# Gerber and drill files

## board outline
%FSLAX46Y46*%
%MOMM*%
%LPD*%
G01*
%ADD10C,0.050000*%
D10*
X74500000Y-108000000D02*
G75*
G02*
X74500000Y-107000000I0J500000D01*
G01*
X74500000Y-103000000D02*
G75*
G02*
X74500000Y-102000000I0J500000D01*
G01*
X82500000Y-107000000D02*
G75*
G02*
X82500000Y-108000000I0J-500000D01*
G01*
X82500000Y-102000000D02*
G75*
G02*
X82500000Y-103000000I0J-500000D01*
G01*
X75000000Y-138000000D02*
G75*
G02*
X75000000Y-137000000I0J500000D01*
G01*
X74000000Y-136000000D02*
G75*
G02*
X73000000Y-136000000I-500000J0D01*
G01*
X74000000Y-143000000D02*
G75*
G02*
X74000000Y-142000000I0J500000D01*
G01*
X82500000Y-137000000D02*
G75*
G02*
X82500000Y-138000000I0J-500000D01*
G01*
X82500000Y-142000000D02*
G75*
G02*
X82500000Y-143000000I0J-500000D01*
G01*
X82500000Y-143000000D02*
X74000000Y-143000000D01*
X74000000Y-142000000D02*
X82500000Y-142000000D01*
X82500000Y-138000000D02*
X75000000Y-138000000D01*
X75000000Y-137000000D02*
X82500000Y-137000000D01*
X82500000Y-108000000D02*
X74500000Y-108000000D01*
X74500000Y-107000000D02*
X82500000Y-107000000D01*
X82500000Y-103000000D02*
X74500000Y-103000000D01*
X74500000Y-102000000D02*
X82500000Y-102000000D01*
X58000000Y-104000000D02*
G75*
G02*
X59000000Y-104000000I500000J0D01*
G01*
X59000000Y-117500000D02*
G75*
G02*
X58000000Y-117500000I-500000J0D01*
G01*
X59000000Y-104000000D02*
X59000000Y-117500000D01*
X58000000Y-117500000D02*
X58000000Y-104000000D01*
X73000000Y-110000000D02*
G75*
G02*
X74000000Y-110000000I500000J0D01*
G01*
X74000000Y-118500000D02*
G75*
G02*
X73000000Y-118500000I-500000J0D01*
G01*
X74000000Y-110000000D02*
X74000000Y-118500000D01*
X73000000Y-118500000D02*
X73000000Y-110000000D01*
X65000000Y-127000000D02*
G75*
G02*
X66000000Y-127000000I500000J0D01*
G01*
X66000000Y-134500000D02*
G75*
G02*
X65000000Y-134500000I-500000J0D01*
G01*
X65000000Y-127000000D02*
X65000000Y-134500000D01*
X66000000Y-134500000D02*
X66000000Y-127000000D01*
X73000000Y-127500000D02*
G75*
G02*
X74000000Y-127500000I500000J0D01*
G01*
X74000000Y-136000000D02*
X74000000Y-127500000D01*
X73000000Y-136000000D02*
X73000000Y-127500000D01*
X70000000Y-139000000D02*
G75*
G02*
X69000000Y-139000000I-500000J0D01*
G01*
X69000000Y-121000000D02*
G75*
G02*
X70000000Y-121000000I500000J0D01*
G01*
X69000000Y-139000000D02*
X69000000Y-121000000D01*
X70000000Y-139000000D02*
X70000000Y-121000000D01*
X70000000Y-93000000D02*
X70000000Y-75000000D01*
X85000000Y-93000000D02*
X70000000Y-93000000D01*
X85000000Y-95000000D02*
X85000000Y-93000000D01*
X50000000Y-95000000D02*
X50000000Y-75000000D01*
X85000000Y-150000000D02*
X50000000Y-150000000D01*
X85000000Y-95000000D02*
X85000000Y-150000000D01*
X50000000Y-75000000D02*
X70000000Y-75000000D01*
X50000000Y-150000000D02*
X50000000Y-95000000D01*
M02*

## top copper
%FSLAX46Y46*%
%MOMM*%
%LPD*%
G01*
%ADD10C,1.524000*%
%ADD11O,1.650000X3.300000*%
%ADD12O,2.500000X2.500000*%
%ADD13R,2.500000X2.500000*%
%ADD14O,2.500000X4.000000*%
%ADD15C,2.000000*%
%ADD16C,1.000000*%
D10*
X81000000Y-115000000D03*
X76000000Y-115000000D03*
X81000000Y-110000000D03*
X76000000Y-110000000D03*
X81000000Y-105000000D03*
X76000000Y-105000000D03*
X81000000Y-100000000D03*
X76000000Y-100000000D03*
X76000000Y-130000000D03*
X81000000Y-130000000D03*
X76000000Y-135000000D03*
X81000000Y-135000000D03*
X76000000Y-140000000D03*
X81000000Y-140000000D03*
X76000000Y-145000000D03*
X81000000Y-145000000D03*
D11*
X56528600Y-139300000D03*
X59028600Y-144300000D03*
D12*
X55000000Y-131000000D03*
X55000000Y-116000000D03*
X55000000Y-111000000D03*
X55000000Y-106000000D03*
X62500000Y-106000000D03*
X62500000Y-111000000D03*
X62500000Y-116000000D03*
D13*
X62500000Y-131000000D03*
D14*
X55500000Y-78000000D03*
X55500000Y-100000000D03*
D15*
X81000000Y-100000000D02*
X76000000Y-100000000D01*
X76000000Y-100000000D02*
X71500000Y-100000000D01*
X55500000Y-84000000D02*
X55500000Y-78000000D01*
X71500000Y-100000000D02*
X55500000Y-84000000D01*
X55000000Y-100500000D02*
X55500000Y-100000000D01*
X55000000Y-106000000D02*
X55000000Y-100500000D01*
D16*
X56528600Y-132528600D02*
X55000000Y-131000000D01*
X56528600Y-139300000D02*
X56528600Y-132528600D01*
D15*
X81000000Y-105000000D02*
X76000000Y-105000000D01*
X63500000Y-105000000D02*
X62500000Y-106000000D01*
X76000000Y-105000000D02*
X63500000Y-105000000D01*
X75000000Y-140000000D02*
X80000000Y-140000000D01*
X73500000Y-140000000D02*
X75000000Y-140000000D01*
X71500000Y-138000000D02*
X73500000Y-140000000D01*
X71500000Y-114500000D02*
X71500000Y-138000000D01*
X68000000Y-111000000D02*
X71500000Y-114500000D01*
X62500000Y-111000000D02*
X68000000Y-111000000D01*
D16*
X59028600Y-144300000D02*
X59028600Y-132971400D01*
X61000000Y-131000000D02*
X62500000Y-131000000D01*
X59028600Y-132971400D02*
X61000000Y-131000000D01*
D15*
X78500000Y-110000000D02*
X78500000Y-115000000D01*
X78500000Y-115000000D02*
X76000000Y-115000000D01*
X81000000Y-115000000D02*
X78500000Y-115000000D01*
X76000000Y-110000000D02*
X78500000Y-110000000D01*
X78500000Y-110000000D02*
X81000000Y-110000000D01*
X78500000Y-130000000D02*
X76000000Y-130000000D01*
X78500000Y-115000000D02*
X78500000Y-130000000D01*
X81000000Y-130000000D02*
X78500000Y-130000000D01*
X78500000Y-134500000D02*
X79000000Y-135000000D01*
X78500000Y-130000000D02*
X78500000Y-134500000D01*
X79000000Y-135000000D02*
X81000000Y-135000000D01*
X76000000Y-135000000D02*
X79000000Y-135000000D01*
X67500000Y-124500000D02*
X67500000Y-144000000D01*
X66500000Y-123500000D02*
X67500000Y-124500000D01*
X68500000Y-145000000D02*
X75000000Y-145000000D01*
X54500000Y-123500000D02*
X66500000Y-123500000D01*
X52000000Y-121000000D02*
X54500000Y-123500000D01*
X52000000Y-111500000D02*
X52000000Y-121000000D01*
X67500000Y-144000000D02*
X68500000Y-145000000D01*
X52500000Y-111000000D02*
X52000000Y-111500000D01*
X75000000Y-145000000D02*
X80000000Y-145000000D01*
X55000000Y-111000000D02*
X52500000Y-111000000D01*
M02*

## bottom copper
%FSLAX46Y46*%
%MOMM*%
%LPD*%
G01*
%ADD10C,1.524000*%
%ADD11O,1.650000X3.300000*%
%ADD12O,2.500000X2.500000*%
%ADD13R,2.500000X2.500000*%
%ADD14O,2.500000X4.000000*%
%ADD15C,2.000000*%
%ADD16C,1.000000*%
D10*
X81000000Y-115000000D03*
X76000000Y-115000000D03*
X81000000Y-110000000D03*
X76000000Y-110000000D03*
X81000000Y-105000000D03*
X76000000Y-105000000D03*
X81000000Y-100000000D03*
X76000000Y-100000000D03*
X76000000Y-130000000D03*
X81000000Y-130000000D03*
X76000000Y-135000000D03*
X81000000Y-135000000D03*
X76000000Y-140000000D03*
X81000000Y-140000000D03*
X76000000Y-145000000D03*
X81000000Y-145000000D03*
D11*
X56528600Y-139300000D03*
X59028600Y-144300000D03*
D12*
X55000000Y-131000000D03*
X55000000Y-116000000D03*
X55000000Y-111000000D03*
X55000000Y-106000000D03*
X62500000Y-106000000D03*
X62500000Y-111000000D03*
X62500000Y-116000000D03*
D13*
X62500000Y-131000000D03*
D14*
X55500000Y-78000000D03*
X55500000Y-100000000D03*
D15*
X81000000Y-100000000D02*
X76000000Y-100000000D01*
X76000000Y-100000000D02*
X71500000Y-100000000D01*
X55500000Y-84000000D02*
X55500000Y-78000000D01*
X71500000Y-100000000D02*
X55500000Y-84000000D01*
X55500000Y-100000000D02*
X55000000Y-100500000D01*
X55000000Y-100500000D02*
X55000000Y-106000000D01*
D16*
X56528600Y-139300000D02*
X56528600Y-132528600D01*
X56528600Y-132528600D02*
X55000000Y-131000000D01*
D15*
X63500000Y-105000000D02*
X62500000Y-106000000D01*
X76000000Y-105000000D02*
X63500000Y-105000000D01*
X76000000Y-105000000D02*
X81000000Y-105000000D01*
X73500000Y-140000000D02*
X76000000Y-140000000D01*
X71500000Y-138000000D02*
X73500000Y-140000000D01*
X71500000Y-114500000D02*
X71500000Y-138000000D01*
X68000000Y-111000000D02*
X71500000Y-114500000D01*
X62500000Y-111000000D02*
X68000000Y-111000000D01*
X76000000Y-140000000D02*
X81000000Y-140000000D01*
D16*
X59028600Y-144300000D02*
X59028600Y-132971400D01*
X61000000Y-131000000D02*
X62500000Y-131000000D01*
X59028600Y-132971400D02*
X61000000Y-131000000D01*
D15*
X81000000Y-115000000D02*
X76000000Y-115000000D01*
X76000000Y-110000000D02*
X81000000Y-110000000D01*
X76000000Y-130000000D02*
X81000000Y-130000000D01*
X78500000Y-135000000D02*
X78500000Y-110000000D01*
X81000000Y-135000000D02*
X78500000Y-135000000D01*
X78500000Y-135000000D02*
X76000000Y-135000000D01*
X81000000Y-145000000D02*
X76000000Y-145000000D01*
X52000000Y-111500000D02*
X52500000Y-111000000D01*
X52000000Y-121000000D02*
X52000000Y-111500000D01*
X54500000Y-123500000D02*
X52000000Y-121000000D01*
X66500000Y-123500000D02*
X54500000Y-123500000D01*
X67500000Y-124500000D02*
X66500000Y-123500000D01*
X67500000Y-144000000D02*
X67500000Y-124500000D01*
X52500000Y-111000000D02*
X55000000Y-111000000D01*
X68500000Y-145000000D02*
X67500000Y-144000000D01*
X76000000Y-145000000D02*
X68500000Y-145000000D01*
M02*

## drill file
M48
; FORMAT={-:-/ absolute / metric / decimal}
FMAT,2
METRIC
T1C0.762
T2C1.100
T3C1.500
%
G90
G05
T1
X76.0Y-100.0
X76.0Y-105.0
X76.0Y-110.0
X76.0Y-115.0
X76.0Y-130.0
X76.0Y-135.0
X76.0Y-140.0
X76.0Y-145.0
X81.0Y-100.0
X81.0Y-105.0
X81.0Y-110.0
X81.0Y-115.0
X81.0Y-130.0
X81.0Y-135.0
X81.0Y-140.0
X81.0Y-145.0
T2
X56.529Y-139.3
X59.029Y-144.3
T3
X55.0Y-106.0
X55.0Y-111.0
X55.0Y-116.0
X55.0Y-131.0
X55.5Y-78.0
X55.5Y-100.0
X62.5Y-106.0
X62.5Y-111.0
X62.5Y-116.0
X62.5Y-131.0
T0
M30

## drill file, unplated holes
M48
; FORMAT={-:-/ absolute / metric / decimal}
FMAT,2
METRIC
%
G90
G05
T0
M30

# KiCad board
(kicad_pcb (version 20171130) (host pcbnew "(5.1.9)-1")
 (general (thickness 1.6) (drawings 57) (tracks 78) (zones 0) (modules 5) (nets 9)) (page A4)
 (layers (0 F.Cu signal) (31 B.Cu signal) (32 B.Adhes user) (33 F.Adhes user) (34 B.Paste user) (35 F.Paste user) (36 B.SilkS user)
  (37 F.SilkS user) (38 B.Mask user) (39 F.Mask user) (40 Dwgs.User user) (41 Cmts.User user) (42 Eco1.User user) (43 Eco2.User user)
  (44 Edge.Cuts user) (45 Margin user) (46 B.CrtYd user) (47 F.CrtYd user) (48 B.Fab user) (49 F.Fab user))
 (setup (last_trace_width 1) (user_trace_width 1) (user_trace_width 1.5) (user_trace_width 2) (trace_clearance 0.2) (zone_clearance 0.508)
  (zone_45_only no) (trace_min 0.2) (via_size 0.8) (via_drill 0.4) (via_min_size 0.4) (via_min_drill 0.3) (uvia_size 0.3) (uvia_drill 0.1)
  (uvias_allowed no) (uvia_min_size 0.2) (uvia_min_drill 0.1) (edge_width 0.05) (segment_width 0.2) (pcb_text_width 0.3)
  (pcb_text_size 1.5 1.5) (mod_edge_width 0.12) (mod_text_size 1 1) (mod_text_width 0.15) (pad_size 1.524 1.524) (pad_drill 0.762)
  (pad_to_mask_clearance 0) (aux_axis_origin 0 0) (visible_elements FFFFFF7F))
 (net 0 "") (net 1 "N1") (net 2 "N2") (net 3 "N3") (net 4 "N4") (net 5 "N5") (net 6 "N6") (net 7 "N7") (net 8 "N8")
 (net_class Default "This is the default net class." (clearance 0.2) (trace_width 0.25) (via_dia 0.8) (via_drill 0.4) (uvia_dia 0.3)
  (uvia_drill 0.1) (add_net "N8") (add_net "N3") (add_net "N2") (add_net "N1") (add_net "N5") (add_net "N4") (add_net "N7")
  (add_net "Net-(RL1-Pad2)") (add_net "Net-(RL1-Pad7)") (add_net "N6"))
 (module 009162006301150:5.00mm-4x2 (layer F.Cu) (at 76 100 270)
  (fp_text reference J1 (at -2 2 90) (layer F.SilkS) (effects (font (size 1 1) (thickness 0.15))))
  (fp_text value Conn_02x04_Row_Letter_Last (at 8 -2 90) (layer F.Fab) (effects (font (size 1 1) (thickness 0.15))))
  (pad 4b thru_hole circle (at 15 -5 270) (size 1.524 1.524) (drill 0.762) (layers *.Cu *.Mask) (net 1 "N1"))
  (pad 4a thru_hole circle (at 15 0 270) (size 1.524 1.524) (drill 0.762) (layers *.Cu *.Mask) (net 1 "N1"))
  (pad 3b thru_hole circle (at 10 -5 270) (size 1.524 1.524) (drill 0.762) (layers *.Cu *.Mask) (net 1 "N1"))
  (pad 3a thru_hole circle (at 10 0 270) (size 1.524 1.524) (drill 0.762) (layers *.Cu *.Mask) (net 1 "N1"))
  (pad 2b thru_hole circle (at 5 -5 270) (size 1.524 1.524) (drill 0.762) (layers *.Cu *.Mask) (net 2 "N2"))
  (pad 2a thru_hole circle (at 5 0 270) (size 1.524 1.524) (drill 0.762) (layers *.Cu *.Mask) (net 2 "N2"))
  (pad 1b thru_hole circle (at 0 -5 270) (size 1.524 1.524) (drill 0.762) (layers *.Cu *.Mask) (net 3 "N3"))
  (pad 1a thru_hole circle (at 0 0 270) (size 1.524 1.524) (drill 0.762) (layers *.Cu *.Mask) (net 3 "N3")))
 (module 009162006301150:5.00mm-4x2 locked (layer F.Cu) (at 81 145 90)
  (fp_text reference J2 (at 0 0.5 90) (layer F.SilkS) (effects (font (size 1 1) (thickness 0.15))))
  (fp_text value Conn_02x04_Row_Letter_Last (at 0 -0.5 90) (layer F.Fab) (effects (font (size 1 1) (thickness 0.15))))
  (pad 4b thru_hole circle (at 15 -5 90) (size 1.524 1.524) (drill 0.762) (layers *.Cu *.Mask) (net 1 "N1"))
  (pad 4a thru_hole circle (at 15 0 90) (size 1.524 1.524) (drill 0.762) (layers *.Cu *.Mask) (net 1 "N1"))
  (pad 3b thru_hole circle (at 10 -5 90) (size 1.524 1.524) (drill 0.762) (layers *.Cu *.Mask) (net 1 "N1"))
  (pad 3a thru_hole circle (at 10 0 90) (size 1.524 1.524) (drill 0.762) (layers *.Cu *.Mask) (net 1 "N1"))
  (pad 2b thru_hole circle (at 5 -5 90) (size 1.524 1.524) (drill 0.762) (layers *.Cu *.Mask) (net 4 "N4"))
  (pad 2a thru_hole circle (at 5 0 90) (size 1.524 1.524) (drill 0.762) (layers *.Cu *.Mask) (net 4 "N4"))
  (pad 1b thru_hole circle (at 0 -5 90) (size 1.524 1.524) (drill 0.762) (layers *.Cu *.Mask) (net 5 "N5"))
  (pad 1a thru_hole circle (at 0 0 90) (size 1.524 1.524) (drill 0.762) (layers *.Cu *.Mask) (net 5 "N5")))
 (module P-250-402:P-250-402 (layer F.Cu) (at 57 143 270)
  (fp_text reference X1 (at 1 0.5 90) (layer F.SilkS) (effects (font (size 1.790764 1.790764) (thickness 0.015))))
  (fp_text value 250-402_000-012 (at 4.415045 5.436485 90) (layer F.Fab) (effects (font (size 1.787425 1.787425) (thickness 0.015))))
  (pad L2 thru_hole oval (at -3.7 0.4714 270) (size 3.3 1.65) (drill 1.1) (layers *.Cu *.Mask) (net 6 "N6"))
  (pad L1 thru_hole oval (at 1.3 -2.0286 270) (size 3.3 1.65) (drill 1.1) (layers *.Cu *.Mask) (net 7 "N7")))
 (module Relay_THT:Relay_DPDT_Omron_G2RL (layer F.Cu) (at 62.5 131 90)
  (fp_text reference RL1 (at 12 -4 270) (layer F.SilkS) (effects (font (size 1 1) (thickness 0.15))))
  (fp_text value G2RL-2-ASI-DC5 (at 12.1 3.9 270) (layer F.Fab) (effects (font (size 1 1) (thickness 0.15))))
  (pad 8 thru_hole oval (at 0 -7.5 180) (size 2.5 2.5) (drill 1.5) (layers *.Cu *.Mask) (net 6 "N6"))
  (pad 7 thru_hole oval (at 15 -7.5 180) (size 2.5 2.5) (drill 1.5) (layers *.Cu *.Mask))
  (pad 6 thru_hole oval (at 20 -7.5 180) (size 2.5 2.5) (drill 1.5) (layers *.Cu *.Mask) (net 5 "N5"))
  (pad 5 thru_hole oval (at 25 -7.5 180) (size 2.5 2.5) (drill 1.5) (layers *.Cu *.Mask) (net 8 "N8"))
  (pad 4 thru_hole oval (at 25 0 180) (size 2.5 2.5) (drill 1.5) (layers *.Cu *.Mask) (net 2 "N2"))
  (pad 3 thru_hole oval (at 20 0 180) (size 2.5 2.5) (drill 1.5) (layers *.Cu *.Mask) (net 4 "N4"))
  (pad 2 thru_hole oval (at 15 0 180) (size 2.5 2.5) (drill 1.5) (layers *.Cu *.Mask))
  (pad 1 thru_hole rect (at 0 0 180) (size 2.5 2.5) (drill 1.5) (layers *.Cu *.Mask) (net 7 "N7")))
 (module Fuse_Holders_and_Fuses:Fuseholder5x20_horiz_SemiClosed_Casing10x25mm (layer F.Cu) (at 55.5 100 90)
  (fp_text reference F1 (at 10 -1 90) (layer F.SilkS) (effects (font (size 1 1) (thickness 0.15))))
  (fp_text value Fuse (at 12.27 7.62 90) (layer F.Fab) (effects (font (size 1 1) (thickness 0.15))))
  (pad 2 thru_hole oval (at 22 0) (size 2.5 4) (drill 1.5) (layers *.Cu *.Mask) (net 3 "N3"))
  (pad 1 thru_hole oval (at 0 0) (size 2.5 4) (drill 1.5) (layers *.Cu *.Mask) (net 8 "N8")))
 (gr_arc (start 74.5 107.5) (end 74.5 107) (angle -180) (layer Edge.Cuts) (width 0.05))
 (gr_arc (start 74.5 102.5) (end 74.5 102) (angle -180) (layer Edge.Cuts) (width 0.05))
 (gr_arc (start 82.5 107.5) (end 82.5 108) (angle -180) (layer Edge.Cuts) (width 0.05))
 (gr_arc (start 82.5 102.5) (end 82.5 103) (angle -180) (layer Edge.Cuts) (width 0.05))
 (gr_arc (start 75 137.5) (end 75 137) (angle -180) (layer Edge.Cuts) (width 0.05))
 (gr_arc (start 73.5 136) (end 73 136) (angle -180) (layer Edge.Cuts) (width 0.05))
 (gr_arc (start 74 142.5) (end 74 142) (angle -180) (layer Edge.Cuts) (width 0.05))
 (gr_arc (start 82.5 137.5) (end 82.5 138) (angle -180) (layer Edge.Cuts) (width 0.05))
 (gr_arc (start 82.5 142.5) (end 82.5 143) (angle -180) (layer Edge.Cuts) (width 0.05))
 (gr_line (start 82.5 143) (end 74 143) (layer Edge.Cuts) (width 0.05))
 (gr_line (start 74 142) (end 82.5 142) (layer Edge.Cuts) (width 0.05))
 (gr_line (start 82.5 138) (end 75 138) (layer Edge.Cuts) (width 0.05))
 (gr_line (start 75 137) (end 82.5 137) (layer Edge.Cuts) (width 0.05))
 (gr_line (start 82.5 108) (end 74.5 108) (layer Edge.Cuts) (width 0.05))
 (gr_line (start 74.5 107) (end 82.5 107) (layer Edge.Cuts) (width 0.05))
 (gr_line (start 82.5 103) (end 74.5 103) (layer Edge.Cuts) (width 0.05))
 (gr_line (start 74.5 102) (end 82.5 102) (layer Edge.Cuts) (width 0.05))
 (gr_arc (start 58.5 104) (end 59 104) (angle -180) (layer Edge.Cuts) (width 0.05))
 (gr_arc (start 58.5 117.5) (end 58 117.5) (angle -180) (layer Edge.Cuts) (width 0.05))
 (gr_line (start 59 104) (end 59 117.5) (layer Edge.Cuts) (width 0.05))
 (gr_line (start 58 117.5) (end 58 104) (layer Edge.Cuts) (width 0.05))
 (gr_arc (start 73.5 110) (end 74 110) (angle -180) (layer Edge.Cuts) (width 0.05))
 (gr_arc (start 73.5 118.5) (end 73 118.5) (angle -180) (layer Edge.Cuts) (width 0.05))
 (gr_line (start 74 110) (end 74 118.5) (layer Edge.Cuts) (width 0.05))
 (gr_line (start 73 118.5) (end 73 110) (layer Edge.Cuts) (width 0.05))
 (gr_arc (start 65.5 127) (end 66 127) (angle -180) (layer Edge.Cuts) (width 0.05))
 (gr_arc (start 65.5 134.5) (end 65 134.5) (angle -180) (layer Edge.Cuts) (width 0.05))
 (gr_line (start 65 127) (end 65 134.5) (layer Edge.Cuts) (width 0.05))
 (gr_line (start 66 134.5) (end 66 127) (layer Edge.Cuts) (width 0.05))
 (gr_arc (start 73.5 127.5) (end 74 127.5) (angle -180) (layer Edge.Cuts) (width 0.05))
 (gr_line (start 74 136) (end 74 127.5) (layer Edge.Cuts) (width 0.05))
 (gr_line (start 73 136) (end 73 127.5) (layer Edge.Cuts) (width 0.05))
 (gr_arc (start 69.5 139) (end 69 139) (angle -180) (layer Edge.Cuts) (width 0.05))
 (gr_arc (start 69.5 121) (end 70 121) (angle -180) (layer Edge.Cuts) (width 0.05))
 (gr_line (start 69 139) (end 69 121) (layer Edge.Cuts) (width 0.05))
 (gr_line (start 70 139) (end 70 121) (layer Edge.Cuts) (width 0.05))
 (gr_line (start 70 93) (end 70 75) (layer Edge.Cuts) (width 0.05))
 (gr_line (start 85 93) (end 70 93) (layer Edge.Cuts) (width 0.05))
 (gr_line (start 85 95) (end 85 93) (layer Edge.Cuts) (width 0.05))
 (gr_line (start 50 95) (end 50 75) (layer Edge.Cuts) (width 0.05))
 (gr_line (start 85 150) (end 50 150) (layer Edge.Cuts) (width 0.05))
 (gr_line (start 85 95) (end 85 150) (layer Edge.Cuts) (width 0.05))
 (gr_line (start 50 75) (end 70 75) (layer Edge.Cuts) (width 0.05))
 (gr_line (start 50 150) (end 50 95) (layer Edge.Cuts) (width 0.05))
 (segment (start 81 100) (end 76 100) (width 2) (layer B.Cu) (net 3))
 (segment (start 76 100) (end 71.5 100) (width 2) (layer B.Cu) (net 3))
 (segment (start 55.5 84) (end 55.5 78) (width 2) (layer B.Cu) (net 3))
 (segment (start 71.5 100) (end 55.5 84) (width 2) (layer B.Cu) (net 3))
 (segment (start 81 100) (end 76 100) (width 2) (layer F.Cu) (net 3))
 (segment (start 76 100) (end 71.5 100) (width 2) (layer F.Cu) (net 3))
 (segment (start 55.5 84) (end 55.5 78) (width 2) (layer F.Cu) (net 3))
 (segment (start 71.5 100) (end 55.5 84) (width 2) (layer F.Cu) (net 3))
 (segment (start 55.5 100) (end 55 100.5) (width 2) (layer B.Cu) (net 8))
 (segment (start 55 100.5) (end 55 106) (width 2) (layer B.Cu) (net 8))
 (segment (start 55 100.5) (end 55.5 100) (width 2) (layer F.Cu) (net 8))
 (segment (start 55 106) (end 55 100.5) (width 2) (layer F.Cu) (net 8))
 (segment (start 56.5286 139.3) (end 56.5286 132.5286) (width 1) (layer B.Cu) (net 6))
 (segment (start 56.5286 132.5286) (end 55 131) (width 1) (layer B.Cu) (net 6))
 (segment (start 56.5286 132.5286) (end 55 131) (width 1) (layer F.Cu) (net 6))
 (segment (start 56.5286 139.3) (end 56.5286 132.5286) (width 1) (layer F.Cu) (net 6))
 (segment (start 63.5 105) (end 62.5 106) (width 2) (layer B.Cu) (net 2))
 (segment (start 76 105) (end 63.5 105) (width 2) (layer B.Cu) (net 2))
 (segment (start 81 105) (end 76 105) (width 2) (layer F.Cu) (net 2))
 (segment (start 63.5 105) (end 62.5 106) (width 2) (layer F.Cu) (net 2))
 (segment (start 76 105) (end 63.5 105) (width 2) (layer F.Cu) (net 2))
 (segment (start 76 105) (end 81 105) (width 2) (layer B.Cu) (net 2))
 (segment (start 75 140) (end 80 140) (width 2) (layer F.Cu) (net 4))
 (segment (start 73.5 140) (end 75 140) (width 2) (layer F.Cu) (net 4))
 (segment (start 71.5 138) (end 73.5 140) (width 2) (layer F.Cu) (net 4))
 (segment (start 71.5 114.5) (end 71.5 138) (width 2) (layer F.Cu) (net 4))
 (segment (start 68 111) (end 71.5 114.5) (width 2) (layer F.Cu) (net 4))
 (segment (start 62.5 111) (end 68 111) (width 2) (layer F.Cu) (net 4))
 (segment (start 73.5 140) (end 76 140) (width 2) (layer B.Cu) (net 4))
 (segment (start 71.5 138) (end 73.5 140) (width 2) (layer B.Cu) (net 4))
 (segment (start 71.5 114.5) (end 71.5 138) (width 2) (layer B.Cu) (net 4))
 (segment (start 68 111) (end 71.5 114.5) (width 2) (layer B.Cu) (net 4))
 (segment (start 62.5 111) (end 68 111) (width 2) (layer B.Cu) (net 4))
 (segment (start 76 140) (end 81 140) (width 2) (layer B.Cu) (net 4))
 (segment (start 59.0286 144.3) (end 59.0286 132.9714) (width 1) (layer F.Cu) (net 7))
 (segment (start 61 131) (end 62.5 131) (width 1) (layer F.Cu) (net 7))
 (segment (start 59.0286 132.9714) (end 61 131) (width 1) (layer F.Cu) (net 7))
 (segment (start 59.0286 144.3) (end 59.0286 132.9714) (width 1) (layer B.Cu) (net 7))
 (segment (start 61 131) (end 62.5 131) (width 1) (layer B.Cu) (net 7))
 (segment (start 59.0286 132.9714) (end 61 131) (width 1) (layer B.Cu) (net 7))
 (segment (start 78.5 110) (end 78.5 115) (width 2) (layer F.Cu) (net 1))
 (segment (start 78.5 115) (end 76 115) (width 2) (layer F.Cu) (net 1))
 (segment (start 81 115) (end 78.5 115) (width 2) (layer F.Cu) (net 1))
 (segment (start 76 110) (end 78.5 110) (width 2) (layer F.Cu) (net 1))
 (segment (start 78.5 110) (end 81 110) (width 2) (layer F.Cu) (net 1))
 (segment (start 78.5 130) (end 76 130) (width 2) (layer F.Cu) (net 1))
 (segment (start 78.5 115) (end 78.5 130) (width 2) (layer F.Cu) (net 1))
 (segment (start 81 130) (end 78.5 130) (width 2) (layer F.Cu) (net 1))
 (segment (start 78.5 134.5) (end 79 135) (width 2) (layer F.Cu) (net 1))
 (segment (start 78.5 130) (end 78.5 134.5) (width 2) (layer F.Cu) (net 1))
 (segment (start 79 135) (end 81 135) (width 2) (layer F.Cu) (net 1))
 (segment (start 76 135) (end 79 135) (width 2) (layer F.Cu) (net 1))
 (segment (start 81 115) (end 76 115) (width 2) (layer B.Cu) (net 1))
 (segment (start 76 110) (end 81 110) (width 2) (layer B.Cu) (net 1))
 (segment (start 76 130) (end 81 130) (width 2) (layer B.Cu) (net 1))
 (segment (start 78.5 135) (end 78.5 110) (width 2) (layer B.Cu) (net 1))
 (segment (start 81 135) (end 78.5 135) (width 2) (layer B.Cu) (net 1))
 (segment (start 78.5 135) (end 76 135) (width 2) (layer B.Cu) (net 1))
 (segment (start 81 145) (end 76 145) (width 2) (layer B.Cu) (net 5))
 (segment (start 67.5 124.5) (end 67.5 144) (width 2) (layer F.Cu) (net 5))
 (segment (start 66.5 123.5) (end 67.5 124.5) (width 2) (layer F.Cu) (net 5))
 (segment (start 68.5 145) (end 75 145) (width 2) (layer F.Cu) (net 5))
 (segment (start 54.5 123.5) (end 66.5 123.5) (width 2) (layer F.Cu) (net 5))
 (segment (start 52 121) (end 54.5 123.5) (width 2) (layer F.Cu) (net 5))
 (segment (start 52 111.5) (end 52 121) (width 2) (layer F.Cu) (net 5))
 (segment (start 67.5 144) (end 68.5 145) (width 2) (layer F.Cu) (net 5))
 (segment (start 52.5 111) (end 52 111.5) (width 2) (layer F.Cu) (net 5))
 (segment (start 75 145) (end 80 145) (width 2) (layer F.Cu) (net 5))
 (segment (start 55 111) (end 52.5 111) (width 2) (layer F.Cu) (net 5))
 (segment (start 52 111.5) (end 52.5 111) (width 2) (layer B.Cu) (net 5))
 (segment (start 52 121) (end 52 111.5) (width 2) (layer B.Cu) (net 5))
 (segment (start 54.5 123.5) (end 52 121) (width 2) (layer B.Cu) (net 5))
 (segment (start 66.5 123.5) (end 54.5 123.5) (width 2) (layer B.Cu) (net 5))
 (segment (start 67.5 124.5) (end 66.5 123.5) (width 2) (layer B.Cu) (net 5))
 (segment (start 67.5 144) (end 67.5 124.5) (width 2) (layer B.Cu) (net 5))
 (segment (start 52.5 111) (end 55 111) (width 2) (layer B.Cu) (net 5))
 (segment (start 68.5 145) (end 67.5 144) (width 2) (layer B.Cu) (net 5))
 (segment (start 76 145) (end 68.5 145) (width 2) (layer B.Cu) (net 5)))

